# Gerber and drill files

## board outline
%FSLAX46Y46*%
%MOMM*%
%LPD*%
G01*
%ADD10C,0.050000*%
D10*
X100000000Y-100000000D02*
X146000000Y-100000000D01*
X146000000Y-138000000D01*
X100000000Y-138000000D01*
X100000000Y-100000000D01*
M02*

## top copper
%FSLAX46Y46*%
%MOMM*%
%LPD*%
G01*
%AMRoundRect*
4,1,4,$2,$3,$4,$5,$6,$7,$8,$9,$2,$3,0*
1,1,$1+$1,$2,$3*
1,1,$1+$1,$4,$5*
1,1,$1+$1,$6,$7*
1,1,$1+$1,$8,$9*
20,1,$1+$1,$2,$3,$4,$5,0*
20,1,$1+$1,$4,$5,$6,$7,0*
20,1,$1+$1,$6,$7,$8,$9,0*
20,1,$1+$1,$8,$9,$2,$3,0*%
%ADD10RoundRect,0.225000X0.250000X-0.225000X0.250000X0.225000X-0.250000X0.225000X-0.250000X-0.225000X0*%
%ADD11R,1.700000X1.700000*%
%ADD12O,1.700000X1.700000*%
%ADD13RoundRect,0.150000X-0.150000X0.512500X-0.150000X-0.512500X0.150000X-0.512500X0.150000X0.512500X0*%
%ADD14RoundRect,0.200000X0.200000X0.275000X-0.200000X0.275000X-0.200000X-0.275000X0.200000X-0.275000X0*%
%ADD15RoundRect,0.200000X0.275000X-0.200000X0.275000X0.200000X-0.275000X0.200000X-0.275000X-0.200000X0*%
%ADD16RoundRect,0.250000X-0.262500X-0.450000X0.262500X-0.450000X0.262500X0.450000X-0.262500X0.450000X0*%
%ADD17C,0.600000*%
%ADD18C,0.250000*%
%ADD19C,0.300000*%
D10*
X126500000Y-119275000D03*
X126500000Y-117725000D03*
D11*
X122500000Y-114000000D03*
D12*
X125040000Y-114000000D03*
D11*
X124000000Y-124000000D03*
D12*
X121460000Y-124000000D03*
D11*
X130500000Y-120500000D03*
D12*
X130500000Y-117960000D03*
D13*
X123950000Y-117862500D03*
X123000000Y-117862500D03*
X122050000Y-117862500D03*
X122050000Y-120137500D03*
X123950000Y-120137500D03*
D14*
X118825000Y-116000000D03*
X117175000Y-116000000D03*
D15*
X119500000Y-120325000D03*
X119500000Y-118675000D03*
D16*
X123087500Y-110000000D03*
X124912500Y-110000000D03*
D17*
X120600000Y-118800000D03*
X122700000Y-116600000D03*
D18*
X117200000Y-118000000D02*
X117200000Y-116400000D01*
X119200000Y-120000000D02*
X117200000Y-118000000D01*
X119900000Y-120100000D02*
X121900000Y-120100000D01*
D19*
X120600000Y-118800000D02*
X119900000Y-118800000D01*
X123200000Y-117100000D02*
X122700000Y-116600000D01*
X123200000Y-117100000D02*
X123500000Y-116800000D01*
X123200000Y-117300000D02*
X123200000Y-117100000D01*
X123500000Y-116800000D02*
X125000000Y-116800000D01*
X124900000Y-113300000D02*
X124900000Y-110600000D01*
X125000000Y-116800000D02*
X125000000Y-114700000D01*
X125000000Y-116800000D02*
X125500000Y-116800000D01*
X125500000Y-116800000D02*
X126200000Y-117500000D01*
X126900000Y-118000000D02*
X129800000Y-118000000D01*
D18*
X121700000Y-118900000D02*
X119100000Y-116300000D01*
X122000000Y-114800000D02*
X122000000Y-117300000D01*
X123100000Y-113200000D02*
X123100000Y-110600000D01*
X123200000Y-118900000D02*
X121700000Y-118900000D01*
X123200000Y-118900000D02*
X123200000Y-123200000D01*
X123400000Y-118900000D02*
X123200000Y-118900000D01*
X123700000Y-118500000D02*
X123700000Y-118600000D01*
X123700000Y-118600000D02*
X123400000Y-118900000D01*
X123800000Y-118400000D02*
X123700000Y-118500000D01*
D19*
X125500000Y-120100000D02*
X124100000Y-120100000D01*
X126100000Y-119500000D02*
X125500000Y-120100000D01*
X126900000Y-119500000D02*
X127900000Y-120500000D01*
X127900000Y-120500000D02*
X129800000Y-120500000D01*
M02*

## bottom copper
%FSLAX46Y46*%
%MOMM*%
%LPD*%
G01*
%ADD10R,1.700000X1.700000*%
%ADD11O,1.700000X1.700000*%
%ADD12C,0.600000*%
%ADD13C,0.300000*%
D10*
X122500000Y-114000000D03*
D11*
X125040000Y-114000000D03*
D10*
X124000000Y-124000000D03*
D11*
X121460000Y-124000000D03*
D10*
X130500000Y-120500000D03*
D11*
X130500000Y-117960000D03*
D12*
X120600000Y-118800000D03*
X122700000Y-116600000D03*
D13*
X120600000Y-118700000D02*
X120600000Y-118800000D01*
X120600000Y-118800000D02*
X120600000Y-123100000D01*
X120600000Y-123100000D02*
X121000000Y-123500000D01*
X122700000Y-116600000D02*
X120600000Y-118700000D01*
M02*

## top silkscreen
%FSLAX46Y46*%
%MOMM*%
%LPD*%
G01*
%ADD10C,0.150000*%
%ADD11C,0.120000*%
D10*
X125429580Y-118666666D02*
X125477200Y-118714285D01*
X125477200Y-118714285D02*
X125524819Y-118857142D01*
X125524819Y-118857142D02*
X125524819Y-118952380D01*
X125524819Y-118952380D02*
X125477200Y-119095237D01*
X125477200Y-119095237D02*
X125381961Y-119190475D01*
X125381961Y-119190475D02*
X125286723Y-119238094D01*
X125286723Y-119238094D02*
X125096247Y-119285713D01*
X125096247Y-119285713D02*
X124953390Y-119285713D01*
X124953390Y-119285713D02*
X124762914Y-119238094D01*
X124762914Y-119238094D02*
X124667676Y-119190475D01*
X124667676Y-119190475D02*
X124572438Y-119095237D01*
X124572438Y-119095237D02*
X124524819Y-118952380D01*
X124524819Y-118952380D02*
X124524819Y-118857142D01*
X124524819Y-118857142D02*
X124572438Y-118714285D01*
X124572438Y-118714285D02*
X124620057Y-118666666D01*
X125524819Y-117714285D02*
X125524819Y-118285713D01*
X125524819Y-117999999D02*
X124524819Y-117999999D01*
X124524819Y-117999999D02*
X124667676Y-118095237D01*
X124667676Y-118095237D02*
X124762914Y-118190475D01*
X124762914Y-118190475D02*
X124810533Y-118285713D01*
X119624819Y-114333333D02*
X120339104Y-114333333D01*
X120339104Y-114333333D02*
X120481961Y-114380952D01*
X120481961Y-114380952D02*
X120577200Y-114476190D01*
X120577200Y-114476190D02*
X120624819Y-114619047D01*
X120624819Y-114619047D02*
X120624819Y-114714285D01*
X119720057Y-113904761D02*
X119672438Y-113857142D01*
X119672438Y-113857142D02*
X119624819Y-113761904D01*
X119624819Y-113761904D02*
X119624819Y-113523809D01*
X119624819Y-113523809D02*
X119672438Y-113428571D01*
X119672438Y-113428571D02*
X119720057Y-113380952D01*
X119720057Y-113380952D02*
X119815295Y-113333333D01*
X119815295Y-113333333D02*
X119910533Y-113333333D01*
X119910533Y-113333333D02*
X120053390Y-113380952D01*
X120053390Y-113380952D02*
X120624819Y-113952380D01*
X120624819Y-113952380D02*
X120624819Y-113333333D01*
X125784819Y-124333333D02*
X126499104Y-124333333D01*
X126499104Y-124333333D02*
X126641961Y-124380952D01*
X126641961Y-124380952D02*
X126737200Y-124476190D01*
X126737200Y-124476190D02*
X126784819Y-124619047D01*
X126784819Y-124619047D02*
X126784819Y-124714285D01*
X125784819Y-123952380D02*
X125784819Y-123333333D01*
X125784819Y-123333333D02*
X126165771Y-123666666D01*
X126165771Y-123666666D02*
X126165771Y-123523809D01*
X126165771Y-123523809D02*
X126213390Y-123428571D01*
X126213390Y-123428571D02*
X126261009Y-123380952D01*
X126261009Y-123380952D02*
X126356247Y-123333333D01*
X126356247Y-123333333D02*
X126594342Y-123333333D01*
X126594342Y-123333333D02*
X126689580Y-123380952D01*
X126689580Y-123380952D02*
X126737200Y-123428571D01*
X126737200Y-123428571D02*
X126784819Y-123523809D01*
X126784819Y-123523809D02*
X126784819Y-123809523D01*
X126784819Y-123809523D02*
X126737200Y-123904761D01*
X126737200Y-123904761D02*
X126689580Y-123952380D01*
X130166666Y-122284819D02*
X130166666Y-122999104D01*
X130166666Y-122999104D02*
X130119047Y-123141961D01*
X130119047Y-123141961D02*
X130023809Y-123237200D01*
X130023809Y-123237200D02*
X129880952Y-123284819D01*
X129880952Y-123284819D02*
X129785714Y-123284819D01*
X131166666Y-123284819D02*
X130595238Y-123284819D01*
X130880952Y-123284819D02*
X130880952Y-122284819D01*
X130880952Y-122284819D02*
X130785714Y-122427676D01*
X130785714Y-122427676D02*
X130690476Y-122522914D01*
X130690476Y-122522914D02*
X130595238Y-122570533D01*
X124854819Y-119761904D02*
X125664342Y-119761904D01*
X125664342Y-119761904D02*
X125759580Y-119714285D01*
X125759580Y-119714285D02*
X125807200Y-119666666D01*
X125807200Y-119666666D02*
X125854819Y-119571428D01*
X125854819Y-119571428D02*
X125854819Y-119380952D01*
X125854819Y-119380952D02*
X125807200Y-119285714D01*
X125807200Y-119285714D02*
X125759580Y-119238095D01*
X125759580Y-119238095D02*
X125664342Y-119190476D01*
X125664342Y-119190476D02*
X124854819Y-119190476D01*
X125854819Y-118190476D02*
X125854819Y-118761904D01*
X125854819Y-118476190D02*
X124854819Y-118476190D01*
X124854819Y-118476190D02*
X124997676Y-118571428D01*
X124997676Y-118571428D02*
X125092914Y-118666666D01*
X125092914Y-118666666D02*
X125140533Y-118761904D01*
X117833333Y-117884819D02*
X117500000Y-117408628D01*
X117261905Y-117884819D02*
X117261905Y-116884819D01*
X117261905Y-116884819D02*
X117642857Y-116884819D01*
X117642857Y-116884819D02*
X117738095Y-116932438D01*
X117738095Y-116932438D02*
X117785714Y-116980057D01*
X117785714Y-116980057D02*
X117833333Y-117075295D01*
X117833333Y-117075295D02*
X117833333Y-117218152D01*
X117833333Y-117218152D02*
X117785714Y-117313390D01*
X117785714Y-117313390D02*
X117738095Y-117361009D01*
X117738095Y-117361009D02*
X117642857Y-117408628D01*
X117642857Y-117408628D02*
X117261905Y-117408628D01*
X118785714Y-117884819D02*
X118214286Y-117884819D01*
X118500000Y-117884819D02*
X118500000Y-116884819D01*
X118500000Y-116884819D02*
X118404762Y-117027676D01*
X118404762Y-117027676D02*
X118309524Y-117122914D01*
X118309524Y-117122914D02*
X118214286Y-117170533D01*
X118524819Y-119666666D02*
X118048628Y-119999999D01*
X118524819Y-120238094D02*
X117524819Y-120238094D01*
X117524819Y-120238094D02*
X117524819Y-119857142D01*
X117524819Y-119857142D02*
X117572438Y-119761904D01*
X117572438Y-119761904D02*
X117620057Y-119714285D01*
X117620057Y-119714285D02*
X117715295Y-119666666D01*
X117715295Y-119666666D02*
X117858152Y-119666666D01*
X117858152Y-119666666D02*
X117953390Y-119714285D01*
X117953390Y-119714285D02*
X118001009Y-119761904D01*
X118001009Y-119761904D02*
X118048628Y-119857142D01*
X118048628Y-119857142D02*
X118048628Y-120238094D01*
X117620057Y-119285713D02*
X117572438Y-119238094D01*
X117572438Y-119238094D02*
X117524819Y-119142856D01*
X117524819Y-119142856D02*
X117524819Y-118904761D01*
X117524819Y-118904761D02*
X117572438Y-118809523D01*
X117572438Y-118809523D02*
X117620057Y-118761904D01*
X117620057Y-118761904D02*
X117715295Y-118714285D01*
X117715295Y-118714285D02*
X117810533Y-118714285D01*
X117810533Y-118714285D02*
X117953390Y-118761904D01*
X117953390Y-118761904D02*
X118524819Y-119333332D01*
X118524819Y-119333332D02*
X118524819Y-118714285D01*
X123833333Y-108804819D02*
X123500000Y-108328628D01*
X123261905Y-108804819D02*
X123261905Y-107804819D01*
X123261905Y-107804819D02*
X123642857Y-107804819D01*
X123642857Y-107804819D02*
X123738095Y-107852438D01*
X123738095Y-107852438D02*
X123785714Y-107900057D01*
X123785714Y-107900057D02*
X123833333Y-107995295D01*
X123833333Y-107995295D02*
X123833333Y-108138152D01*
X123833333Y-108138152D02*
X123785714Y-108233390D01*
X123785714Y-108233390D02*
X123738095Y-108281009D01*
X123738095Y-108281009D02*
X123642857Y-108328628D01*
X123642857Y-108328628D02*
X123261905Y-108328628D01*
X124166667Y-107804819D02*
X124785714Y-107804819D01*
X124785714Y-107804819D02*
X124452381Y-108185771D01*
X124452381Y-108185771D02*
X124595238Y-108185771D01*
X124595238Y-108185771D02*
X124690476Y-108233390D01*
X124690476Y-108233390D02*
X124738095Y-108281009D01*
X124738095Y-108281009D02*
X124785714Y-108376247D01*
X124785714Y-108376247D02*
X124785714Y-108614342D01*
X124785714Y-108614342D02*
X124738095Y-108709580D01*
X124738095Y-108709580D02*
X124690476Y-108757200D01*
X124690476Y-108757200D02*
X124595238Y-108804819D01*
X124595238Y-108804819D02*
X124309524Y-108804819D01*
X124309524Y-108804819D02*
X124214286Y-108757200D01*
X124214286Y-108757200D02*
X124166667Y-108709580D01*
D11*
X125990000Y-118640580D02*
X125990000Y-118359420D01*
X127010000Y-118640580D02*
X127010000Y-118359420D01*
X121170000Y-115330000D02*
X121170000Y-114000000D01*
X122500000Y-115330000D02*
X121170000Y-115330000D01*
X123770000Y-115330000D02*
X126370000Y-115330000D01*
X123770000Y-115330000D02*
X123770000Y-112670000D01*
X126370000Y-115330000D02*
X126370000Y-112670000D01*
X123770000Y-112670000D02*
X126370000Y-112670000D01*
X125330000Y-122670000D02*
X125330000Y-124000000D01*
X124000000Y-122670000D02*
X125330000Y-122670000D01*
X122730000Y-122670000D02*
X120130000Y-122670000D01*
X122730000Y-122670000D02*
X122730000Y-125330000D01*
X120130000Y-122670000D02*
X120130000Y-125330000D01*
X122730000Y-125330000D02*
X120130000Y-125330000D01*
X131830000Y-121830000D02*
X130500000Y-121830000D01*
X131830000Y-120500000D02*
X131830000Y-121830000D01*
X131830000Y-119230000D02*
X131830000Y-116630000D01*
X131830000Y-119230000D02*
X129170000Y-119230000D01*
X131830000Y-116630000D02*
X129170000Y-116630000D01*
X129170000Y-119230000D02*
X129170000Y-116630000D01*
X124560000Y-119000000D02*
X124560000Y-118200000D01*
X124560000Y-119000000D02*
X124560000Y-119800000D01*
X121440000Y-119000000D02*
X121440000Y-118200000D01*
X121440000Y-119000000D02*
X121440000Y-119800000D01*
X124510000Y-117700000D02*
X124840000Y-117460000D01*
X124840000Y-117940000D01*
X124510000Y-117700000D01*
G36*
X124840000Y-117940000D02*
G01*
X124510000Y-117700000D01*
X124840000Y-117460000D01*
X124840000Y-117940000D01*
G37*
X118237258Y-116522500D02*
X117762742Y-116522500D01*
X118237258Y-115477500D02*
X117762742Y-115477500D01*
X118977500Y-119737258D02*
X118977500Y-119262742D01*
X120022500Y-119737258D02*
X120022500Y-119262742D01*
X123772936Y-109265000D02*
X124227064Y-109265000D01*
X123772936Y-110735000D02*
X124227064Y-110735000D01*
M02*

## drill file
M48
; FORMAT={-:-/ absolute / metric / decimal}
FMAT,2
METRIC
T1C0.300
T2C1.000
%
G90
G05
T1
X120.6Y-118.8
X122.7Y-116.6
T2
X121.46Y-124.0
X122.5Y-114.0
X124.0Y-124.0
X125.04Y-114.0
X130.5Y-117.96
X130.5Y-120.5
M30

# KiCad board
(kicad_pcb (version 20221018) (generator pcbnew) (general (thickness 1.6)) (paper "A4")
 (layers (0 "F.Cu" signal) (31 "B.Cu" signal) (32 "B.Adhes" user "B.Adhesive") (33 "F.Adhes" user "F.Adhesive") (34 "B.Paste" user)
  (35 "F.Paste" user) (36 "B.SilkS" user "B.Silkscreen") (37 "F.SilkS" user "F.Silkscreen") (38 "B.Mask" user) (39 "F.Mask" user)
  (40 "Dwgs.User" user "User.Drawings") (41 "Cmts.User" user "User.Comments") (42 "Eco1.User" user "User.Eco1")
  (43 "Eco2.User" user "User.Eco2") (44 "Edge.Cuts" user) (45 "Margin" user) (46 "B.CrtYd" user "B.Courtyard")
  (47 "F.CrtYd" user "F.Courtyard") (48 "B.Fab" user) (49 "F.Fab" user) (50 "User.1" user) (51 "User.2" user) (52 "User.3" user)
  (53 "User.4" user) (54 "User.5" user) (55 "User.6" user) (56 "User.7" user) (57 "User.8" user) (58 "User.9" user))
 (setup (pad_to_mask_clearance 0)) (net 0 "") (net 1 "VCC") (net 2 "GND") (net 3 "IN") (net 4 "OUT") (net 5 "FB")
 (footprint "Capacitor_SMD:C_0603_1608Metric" (layer "F.Cu") (at 126.5 118.5 90)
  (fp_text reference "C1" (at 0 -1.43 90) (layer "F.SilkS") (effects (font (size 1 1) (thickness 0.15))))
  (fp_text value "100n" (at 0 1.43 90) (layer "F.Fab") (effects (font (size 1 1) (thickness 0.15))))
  (fp_line (start -0.14058 -0.51) (end 0.14058 -0.51) (stroke (width 0.12) (type solid)) (layer "F.SilkS"))
  (fp_line (start -0.14058 0.51) (end 0.14058 0.51) (stroke (width 0.12) (type solid)) (layer "F.SilkS"))
  (pad "1" smd roundrect (at -0.775 0 90) (size 0.9 0.95) (layers "F.Cu" "F.Paste" "F.Mask") (roundrect_rratio 0.25) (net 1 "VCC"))
  (pad "2" smd roundrect (at 0.775 0 90) (size 0.9 0.95) (layers "F.Cu" "F.Paste" "F.Mask") (roundrect_rratio 0.25) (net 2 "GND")))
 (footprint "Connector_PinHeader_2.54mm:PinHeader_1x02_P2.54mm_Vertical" (layer "F.Cu") (at 122.5 114 90)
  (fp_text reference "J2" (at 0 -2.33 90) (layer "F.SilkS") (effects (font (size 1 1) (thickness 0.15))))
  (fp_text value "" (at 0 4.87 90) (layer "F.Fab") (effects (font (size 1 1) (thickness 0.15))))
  (fp_line (start -1.33 -1.33) (end 0 -1.33) (stroke (width 0.12) (type solid)) (layer "F.SilkS"))
  (fp_line (start -1.33 0) (end -1.33 -1.33) (stroke (width 0.12) (type solid)) (layer "F.SilkS"))
  (fp_line (start -1.33 1.27) (end -1.33 3.87) (stroke (width 0.12) (type solid)) (layer "F.SilkS"))
  (fp_line (start -1.33 1.27) (end 1.33 1.27) (stroke (width 0.12) (type solid)) (layer "F.SilkS"))
  (fp_line (start -1.33 3.87) (end 1.33 3.87) (stroke (width 0.12) (type solid)) (layer "F.SilkS"))
  (fp_line (start 1.33 1.27) (end 1.33 3.87) (stroke (width 0.12) (type solid)) (layer "F.SilkS"))
  (pad "1" thru_hole rect (at 0 0 90) (size 1.7 1.7) (drill 1) (layers "*.Cu" "*.Mask") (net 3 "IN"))
  (pad "2" thru_hole oval (at 0 2.54 90) (size 1.7 1.7) (drill 1) (layers "*.Cu" "*.Mask") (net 2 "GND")))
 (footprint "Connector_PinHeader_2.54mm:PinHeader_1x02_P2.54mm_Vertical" (layer "F.Cu") (at 124 124 -90)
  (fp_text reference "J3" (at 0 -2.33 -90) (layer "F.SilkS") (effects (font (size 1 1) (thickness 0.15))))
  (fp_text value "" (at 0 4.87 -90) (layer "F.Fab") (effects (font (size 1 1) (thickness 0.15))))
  (fp_line (start -1.33 -1.33) (end 0 -1.33) (stroke (width 0.12) (type solid)) (layer "F.SilkS"))
  (fp_line (start -1.33 0) (end -1.33 -1.33) (stroke (width 0.12) (type solid)) (layer "F.SilkS"))
  (fp_line (start -1.33 1.27) (end -1.33 3.87) (stroke (width 0.12) (type solid)) (layer "F.SilkS"))
  (fp_line (start -1.33 1.27) (end 1.33 1.27) (stroke (width 0.12) (type solid)) (layer "F.SilkS"))
  (fp_line (start -1.33 3.87) (end 1.33 3.87) (stroke (width 0.12) (type solid)) (layer "F.SilkS"))
  (fp_line (start 1.33 1.27) (end 1.33 3.87) (stroke (width 0.12) (type solid)) (layer "F.SilkS"))
  (pad "1" thru_hole rect (at 0 0 270) (size 1.7 1.7) (drill 1) (layers "*.Cu" "*.Mask") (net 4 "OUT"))
  (pad "2" thru_hole oval (at 0 2.54 270) (size 1.7 1.7) (drill 1) (layers "*.Cu" "*.Mask") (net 2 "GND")))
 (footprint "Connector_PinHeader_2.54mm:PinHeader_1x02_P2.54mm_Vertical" (layer "F.Cu") (at 130.5 120.5 180)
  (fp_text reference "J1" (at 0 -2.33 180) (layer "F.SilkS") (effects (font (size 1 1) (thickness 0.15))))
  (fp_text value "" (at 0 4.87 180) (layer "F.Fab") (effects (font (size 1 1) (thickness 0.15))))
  (fp_line (start -1.33 -1.33) (end 0 -1.33) (stroke (width 0.12) (type solid)) (layer "F.SilkS"))
  (fp_line (start -1.33 0) (end -1.33 -1.33) (stroke (width 0.12) (type solid)) (layer "F.SilkS"))
  (fp_line (start -1.33 1.27) (end -1.33 3.87) (stroke (width 0.12) (type solid)) (layer "F.SilkS"))
  (fp_line (start -1.33 1.27) (end 1.33 1.27) (stroke (width 0.12) (type solid)) (layer "F.SilkS"))
  (fp_line (start -1.33 3.87) (end 1.33 3.87) (stroke (width 0.12) (type solid)) (layer "F.SilkS"))
  (fp_line (start 1.33 1.27) (end 1.33 3.87) (stroke (width 0.12) (type solid)) (layer "F.SilkS"))
  (pad "1" thru_hole rect (at 0 0 180) (size 1.7 1.7) (drill 1) (layers "*.Cu" "*.Mask") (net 1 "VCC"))
  (pad "2" thru_hole oval (at 0 2.54 180) (size 1.7 1.7) (drill 1) (layers "*.Cu" "*.Mask") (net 2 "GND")))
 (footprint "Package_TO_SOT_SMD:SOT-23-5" (layer "F.Cu") (at 123 119 -90)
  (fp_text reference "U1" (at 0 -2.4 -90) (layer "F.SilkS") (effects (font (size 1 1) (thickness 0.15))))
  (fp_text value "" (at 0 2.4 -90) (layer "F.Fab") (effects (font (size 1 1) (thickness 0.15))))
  (fp_line (start 0 -1.56) (end -0.8 -1.56) (stroke (width 0.12) (type solid)) (layer "F.SilkS"))
  (fp_line (start 0 -1.56) (end 0.8 -1.56) (stroke (width 0.12) (type solid)) (layer "F.SilkS"))
  (fp_line (start 0 1.56) (end -0.8 1.56) (stroke (width 0.12) (type solid)) (layer "F.SilkS"))
  (fp_line (start 0 1.56) (end 0.8 1.56) (stroke (width 0.12) (type solid)) (layer "F.SilkS"))
  (fp_poly
   (pts (xy -1.3 -1.51) (xy -1.54 -1.84) (xy -1.06 -1.84) (xy -1.3 -1.51)) (stroke (width 0.12) (type solid)) (fill solid) (layer "F.SilkS"))
  (pad "1" smd roundrect (at -1.1375 -0.95 270) (size 1.325 0.6) (layers "F.Cu" "F.Paste" "F.Mask") (roundrect_rratio 0.25) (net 4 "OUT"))
  (pad "2" smd roundrect (at -1.1375 0 270) (size 1.325 0.6) (layers "F.Cu" "F.Paste" "F.Mask") (roundrect_rratio 0.25) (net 2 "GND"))
  (pad "3" smd roundrect (at -1.1375 0.95 270) (size 1.325 0.6) (layers "F.Cu" "F.Paste" "F.Mask") (roundrect_rratio 0.25) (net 3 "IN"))
  (pad "4" smd roundrect (at 1.1375 0.95 270) (size 1.325 0.6) (layers "F.Cu" "F.Paste" "F.Mask") (roundrect_rratio 0.25) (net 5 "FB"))
  (pad "5" smd roundrect (at 1.1375 -0.95 270) (size 1.325 0.6) (layers "F.Cu" "F.Paste" "F.Mask") (roundrect_rratio 0.25) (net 1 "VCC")))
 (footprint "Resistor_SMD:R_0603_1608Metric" (layer "F.Cu") (at 118 116 180)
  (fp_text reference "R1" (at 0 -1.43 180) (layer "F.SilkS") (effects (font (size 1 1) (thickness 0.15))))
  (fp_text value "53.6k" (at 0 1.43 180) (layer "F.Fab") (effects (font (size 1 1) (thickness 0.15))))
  (fp_line (start -0.237258 -0.5225) (end 0.237258 -0.5225) (stroke (width 0.12) (type solid)) (layer "F.SilkS"))
  (fp_line (start -0.237258 0.5225) (end 0.237258 0.5225) (stroke (width 0.12) (type solid)) (layer "F.SilkS"))
  (pad "1" smd roundrect (at -0.825 0 180) (size 0.8 0.95) (layers "F.Cu" "F.Paste" "F.Mask") (roundrect_rratio 0.25) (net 4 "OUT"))
  (pad "2" smd roundrect (at 0.825 0 180) (size 0.8 0.95) (layers "F.Cu" "F.Paste" "F.Mask") (roundrect_rratio 0.25) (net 5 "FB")))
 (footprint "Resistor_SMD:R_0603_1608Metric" (layer "F.Cu") (at 119.5 119.5 90)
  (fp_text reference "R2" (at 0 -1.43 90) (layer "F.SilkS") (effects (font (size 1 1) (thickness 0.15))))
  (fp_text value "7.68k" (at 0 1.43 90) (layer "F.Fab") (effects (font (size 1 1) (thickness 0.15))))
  (fp_line (start -0.237258 -0.5225) (end 0.237258 -0.5225) (stroke (width 0.12) (type solid)) (layer "F.SilkS"))
  (fp_line (start -0.237258 0.5225) (end 0.237258 0.5225) (stroke (width 0.12) (type solid)) (layer "F.SilkS"))
  (pad "1" smd roundrect (at -0.825 0 90) (size 0.8 0.95) (layers "F.Cu" "F.Paste" "F.Mask") (roundrect_rratio 0.25) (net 5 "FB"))
  (pad "2" smd roundrect (at 0.825 0 90) (size 0.8 0.95) (layers "F.Cu" "F.Paste" "F.Mask") (roundrect_rratio 0.25) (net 2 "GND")))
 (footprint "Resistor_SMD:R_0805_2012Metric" (layer "F.Cu") (at 124 110)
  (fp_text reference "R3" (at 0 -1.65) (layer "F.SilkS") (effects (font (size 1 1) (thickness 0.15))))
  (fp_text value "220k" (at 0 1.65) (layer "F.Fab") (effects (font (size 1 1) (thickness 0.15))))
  (fp_line (start -0.227064 -0.735) (end 0.227064 -0.735) (stroke (width 0.12) (type solid)) (layer "F.SilkS"))
  (fp_line (start -0.227064 0.735) (end 0.227064 0.735) (stroke (width 0.12) (type solid)) (layer "F.SilkS"))
  (pad "1" smd roundrect (at -0.9125 0) (size 1.025 1.4) (layers "F.Cu" "F.Paste" "F.Mask") (roundrect_rratio 0.243902) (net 3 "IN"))
  (pad "2" smd roundrect (at 0.9125 0) (size 1.025 1.4) (layers "F.Cu" "F.Paste" "F.Mask") (roundrect_rratio 0.243902) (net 2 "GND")))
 (gr_rect (start 100 100) (end 146 138) (stroke (width 0.05) (type default)) (fill none) (layer "Edge.Cuts"))
 (segment (start 117.2 118) (end 117.2 116.4) (width 0.25) (layer "F.Cu") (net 5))
 (segment (start 119.2 120) (end 117.2 118) (width 0.25) (layer "F.Cu") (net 5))
 (segment (start 119.9 120.1) (end 121.9 120.1) (width 0.25) (layer "F.Cu") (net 5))
 (segment (start 120.6 118.8) (end 119.9 118.8) (width 0.3) (layer "F.Cu") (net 2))
 (segment (start 123.2 117.1) (end 122.7 116.6) (width 0.3) (layer "F.Cu") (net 2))
 (segment (start 123.2 117.1) (end 123.5 116.8) (width 0.3) (layer "F.Cu") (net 2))
 (segment (start 123.2 117.3) (end 123.2 117.1) (width 0.3) (layer "F.Cu") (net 2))
 (segment (start 123.5 116.8) (end 125 116.8) (width 0.3) (layer "F.Cu") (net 2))
 (segment (start 124.9 113.3) (end 124.9 110.6) (width 0.3) (layer "F.Cu") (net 2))
 (segment (start 125 116.8) (end 125 114.7) (width 0.3) (layer "F.Cu") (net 2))
 (segment (start 125 116.8) (end 125.5 116.8) (width 0.3) (layer "F.Cu") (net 2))
 (segment (start 125.5 116.8) (end 126.2 117.5) (width 0.3) (layer "F.Cu") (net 2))
 (segment (start 126.9 118) (end 129.8 118) (width 0.3) (layer "F.Cu") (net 2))
 (via (at 120.6 118.8) (size 0.6) (drill 0.3) (layers "F.Cu" "B.Cu") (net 2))
 (via (at 122.7 116.6) (size 0.6) (drill 0.3) (layers "F.Cu" "B.Cu") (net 2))
 (segment (start 120.6 118.7) (end 120.6 118.8) (width 0.3) (layer "B.Cu") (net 2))
 (segment (start 120.6 118.8) (end 120.6 123.1) (width 0.3) (layer "B.Cu") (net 2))
 (segment (start 120.6 123.1) (end 121 123.5) (width 0.3) (layer "B.Cu") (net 2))
 (segment (start 121.7 118.9) (end 119.1 116.3) (width 0.25) (layer "F.Cu") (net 4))
 (segment (start 122 114.8) (end 122 117.3) (width 0.25) (layer "F.Cu") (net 3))
 (segment (start 122.7 116.6) (end 120.6 118.7) (width 0.3) (layer "B.Cu") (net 2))
 (segment (start 123.1 113.2) (end 123.1 110.6) (width 0.25) (layer "F.Cu") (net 3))
 (segment (start 123.2 118.9) (end 121.7 118.9) (width 0.25) (layer "F.Cu") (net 4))
 (segment (start 123.2 118.9) (end 123.2 123.2) (width 0.25) (layer "F.Cu") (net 4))
 (segment (start 123.4 118.9) (end 123.2 118.9) (width 0.25) (layer "F.Cu") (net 4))
 (segment (start 123.7 118.5) (end 123.7 118.6) (width 0.25) (layer "F.Cu") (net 4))
 (segment (start 123.7 118.6) (end 123.4 118.9) (width 0.25) (layer "F.Cu") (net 4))
 (segment (start 123.8 118.4) (end 123.7 118.5) (width 0.25) (layer "F.Cu") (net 4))
 (segment (start 125.5 120.1) (end 124.1 120.1) (width 0.3) (layer "F.Cu") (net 1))
 (segment (start 126.1 119.5) (end 125.5 120.1) (width 0.3) (layer "F.Cu") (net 1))
 (segment (start 126.9 119.5) (end 127.9 120.5) (width 0.3) (layer "F.Cu") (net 1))
 (segment (start 127.9 120.5) (end 129.8 120.5) (width 0.3) (layer "F.Cu") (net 1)))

